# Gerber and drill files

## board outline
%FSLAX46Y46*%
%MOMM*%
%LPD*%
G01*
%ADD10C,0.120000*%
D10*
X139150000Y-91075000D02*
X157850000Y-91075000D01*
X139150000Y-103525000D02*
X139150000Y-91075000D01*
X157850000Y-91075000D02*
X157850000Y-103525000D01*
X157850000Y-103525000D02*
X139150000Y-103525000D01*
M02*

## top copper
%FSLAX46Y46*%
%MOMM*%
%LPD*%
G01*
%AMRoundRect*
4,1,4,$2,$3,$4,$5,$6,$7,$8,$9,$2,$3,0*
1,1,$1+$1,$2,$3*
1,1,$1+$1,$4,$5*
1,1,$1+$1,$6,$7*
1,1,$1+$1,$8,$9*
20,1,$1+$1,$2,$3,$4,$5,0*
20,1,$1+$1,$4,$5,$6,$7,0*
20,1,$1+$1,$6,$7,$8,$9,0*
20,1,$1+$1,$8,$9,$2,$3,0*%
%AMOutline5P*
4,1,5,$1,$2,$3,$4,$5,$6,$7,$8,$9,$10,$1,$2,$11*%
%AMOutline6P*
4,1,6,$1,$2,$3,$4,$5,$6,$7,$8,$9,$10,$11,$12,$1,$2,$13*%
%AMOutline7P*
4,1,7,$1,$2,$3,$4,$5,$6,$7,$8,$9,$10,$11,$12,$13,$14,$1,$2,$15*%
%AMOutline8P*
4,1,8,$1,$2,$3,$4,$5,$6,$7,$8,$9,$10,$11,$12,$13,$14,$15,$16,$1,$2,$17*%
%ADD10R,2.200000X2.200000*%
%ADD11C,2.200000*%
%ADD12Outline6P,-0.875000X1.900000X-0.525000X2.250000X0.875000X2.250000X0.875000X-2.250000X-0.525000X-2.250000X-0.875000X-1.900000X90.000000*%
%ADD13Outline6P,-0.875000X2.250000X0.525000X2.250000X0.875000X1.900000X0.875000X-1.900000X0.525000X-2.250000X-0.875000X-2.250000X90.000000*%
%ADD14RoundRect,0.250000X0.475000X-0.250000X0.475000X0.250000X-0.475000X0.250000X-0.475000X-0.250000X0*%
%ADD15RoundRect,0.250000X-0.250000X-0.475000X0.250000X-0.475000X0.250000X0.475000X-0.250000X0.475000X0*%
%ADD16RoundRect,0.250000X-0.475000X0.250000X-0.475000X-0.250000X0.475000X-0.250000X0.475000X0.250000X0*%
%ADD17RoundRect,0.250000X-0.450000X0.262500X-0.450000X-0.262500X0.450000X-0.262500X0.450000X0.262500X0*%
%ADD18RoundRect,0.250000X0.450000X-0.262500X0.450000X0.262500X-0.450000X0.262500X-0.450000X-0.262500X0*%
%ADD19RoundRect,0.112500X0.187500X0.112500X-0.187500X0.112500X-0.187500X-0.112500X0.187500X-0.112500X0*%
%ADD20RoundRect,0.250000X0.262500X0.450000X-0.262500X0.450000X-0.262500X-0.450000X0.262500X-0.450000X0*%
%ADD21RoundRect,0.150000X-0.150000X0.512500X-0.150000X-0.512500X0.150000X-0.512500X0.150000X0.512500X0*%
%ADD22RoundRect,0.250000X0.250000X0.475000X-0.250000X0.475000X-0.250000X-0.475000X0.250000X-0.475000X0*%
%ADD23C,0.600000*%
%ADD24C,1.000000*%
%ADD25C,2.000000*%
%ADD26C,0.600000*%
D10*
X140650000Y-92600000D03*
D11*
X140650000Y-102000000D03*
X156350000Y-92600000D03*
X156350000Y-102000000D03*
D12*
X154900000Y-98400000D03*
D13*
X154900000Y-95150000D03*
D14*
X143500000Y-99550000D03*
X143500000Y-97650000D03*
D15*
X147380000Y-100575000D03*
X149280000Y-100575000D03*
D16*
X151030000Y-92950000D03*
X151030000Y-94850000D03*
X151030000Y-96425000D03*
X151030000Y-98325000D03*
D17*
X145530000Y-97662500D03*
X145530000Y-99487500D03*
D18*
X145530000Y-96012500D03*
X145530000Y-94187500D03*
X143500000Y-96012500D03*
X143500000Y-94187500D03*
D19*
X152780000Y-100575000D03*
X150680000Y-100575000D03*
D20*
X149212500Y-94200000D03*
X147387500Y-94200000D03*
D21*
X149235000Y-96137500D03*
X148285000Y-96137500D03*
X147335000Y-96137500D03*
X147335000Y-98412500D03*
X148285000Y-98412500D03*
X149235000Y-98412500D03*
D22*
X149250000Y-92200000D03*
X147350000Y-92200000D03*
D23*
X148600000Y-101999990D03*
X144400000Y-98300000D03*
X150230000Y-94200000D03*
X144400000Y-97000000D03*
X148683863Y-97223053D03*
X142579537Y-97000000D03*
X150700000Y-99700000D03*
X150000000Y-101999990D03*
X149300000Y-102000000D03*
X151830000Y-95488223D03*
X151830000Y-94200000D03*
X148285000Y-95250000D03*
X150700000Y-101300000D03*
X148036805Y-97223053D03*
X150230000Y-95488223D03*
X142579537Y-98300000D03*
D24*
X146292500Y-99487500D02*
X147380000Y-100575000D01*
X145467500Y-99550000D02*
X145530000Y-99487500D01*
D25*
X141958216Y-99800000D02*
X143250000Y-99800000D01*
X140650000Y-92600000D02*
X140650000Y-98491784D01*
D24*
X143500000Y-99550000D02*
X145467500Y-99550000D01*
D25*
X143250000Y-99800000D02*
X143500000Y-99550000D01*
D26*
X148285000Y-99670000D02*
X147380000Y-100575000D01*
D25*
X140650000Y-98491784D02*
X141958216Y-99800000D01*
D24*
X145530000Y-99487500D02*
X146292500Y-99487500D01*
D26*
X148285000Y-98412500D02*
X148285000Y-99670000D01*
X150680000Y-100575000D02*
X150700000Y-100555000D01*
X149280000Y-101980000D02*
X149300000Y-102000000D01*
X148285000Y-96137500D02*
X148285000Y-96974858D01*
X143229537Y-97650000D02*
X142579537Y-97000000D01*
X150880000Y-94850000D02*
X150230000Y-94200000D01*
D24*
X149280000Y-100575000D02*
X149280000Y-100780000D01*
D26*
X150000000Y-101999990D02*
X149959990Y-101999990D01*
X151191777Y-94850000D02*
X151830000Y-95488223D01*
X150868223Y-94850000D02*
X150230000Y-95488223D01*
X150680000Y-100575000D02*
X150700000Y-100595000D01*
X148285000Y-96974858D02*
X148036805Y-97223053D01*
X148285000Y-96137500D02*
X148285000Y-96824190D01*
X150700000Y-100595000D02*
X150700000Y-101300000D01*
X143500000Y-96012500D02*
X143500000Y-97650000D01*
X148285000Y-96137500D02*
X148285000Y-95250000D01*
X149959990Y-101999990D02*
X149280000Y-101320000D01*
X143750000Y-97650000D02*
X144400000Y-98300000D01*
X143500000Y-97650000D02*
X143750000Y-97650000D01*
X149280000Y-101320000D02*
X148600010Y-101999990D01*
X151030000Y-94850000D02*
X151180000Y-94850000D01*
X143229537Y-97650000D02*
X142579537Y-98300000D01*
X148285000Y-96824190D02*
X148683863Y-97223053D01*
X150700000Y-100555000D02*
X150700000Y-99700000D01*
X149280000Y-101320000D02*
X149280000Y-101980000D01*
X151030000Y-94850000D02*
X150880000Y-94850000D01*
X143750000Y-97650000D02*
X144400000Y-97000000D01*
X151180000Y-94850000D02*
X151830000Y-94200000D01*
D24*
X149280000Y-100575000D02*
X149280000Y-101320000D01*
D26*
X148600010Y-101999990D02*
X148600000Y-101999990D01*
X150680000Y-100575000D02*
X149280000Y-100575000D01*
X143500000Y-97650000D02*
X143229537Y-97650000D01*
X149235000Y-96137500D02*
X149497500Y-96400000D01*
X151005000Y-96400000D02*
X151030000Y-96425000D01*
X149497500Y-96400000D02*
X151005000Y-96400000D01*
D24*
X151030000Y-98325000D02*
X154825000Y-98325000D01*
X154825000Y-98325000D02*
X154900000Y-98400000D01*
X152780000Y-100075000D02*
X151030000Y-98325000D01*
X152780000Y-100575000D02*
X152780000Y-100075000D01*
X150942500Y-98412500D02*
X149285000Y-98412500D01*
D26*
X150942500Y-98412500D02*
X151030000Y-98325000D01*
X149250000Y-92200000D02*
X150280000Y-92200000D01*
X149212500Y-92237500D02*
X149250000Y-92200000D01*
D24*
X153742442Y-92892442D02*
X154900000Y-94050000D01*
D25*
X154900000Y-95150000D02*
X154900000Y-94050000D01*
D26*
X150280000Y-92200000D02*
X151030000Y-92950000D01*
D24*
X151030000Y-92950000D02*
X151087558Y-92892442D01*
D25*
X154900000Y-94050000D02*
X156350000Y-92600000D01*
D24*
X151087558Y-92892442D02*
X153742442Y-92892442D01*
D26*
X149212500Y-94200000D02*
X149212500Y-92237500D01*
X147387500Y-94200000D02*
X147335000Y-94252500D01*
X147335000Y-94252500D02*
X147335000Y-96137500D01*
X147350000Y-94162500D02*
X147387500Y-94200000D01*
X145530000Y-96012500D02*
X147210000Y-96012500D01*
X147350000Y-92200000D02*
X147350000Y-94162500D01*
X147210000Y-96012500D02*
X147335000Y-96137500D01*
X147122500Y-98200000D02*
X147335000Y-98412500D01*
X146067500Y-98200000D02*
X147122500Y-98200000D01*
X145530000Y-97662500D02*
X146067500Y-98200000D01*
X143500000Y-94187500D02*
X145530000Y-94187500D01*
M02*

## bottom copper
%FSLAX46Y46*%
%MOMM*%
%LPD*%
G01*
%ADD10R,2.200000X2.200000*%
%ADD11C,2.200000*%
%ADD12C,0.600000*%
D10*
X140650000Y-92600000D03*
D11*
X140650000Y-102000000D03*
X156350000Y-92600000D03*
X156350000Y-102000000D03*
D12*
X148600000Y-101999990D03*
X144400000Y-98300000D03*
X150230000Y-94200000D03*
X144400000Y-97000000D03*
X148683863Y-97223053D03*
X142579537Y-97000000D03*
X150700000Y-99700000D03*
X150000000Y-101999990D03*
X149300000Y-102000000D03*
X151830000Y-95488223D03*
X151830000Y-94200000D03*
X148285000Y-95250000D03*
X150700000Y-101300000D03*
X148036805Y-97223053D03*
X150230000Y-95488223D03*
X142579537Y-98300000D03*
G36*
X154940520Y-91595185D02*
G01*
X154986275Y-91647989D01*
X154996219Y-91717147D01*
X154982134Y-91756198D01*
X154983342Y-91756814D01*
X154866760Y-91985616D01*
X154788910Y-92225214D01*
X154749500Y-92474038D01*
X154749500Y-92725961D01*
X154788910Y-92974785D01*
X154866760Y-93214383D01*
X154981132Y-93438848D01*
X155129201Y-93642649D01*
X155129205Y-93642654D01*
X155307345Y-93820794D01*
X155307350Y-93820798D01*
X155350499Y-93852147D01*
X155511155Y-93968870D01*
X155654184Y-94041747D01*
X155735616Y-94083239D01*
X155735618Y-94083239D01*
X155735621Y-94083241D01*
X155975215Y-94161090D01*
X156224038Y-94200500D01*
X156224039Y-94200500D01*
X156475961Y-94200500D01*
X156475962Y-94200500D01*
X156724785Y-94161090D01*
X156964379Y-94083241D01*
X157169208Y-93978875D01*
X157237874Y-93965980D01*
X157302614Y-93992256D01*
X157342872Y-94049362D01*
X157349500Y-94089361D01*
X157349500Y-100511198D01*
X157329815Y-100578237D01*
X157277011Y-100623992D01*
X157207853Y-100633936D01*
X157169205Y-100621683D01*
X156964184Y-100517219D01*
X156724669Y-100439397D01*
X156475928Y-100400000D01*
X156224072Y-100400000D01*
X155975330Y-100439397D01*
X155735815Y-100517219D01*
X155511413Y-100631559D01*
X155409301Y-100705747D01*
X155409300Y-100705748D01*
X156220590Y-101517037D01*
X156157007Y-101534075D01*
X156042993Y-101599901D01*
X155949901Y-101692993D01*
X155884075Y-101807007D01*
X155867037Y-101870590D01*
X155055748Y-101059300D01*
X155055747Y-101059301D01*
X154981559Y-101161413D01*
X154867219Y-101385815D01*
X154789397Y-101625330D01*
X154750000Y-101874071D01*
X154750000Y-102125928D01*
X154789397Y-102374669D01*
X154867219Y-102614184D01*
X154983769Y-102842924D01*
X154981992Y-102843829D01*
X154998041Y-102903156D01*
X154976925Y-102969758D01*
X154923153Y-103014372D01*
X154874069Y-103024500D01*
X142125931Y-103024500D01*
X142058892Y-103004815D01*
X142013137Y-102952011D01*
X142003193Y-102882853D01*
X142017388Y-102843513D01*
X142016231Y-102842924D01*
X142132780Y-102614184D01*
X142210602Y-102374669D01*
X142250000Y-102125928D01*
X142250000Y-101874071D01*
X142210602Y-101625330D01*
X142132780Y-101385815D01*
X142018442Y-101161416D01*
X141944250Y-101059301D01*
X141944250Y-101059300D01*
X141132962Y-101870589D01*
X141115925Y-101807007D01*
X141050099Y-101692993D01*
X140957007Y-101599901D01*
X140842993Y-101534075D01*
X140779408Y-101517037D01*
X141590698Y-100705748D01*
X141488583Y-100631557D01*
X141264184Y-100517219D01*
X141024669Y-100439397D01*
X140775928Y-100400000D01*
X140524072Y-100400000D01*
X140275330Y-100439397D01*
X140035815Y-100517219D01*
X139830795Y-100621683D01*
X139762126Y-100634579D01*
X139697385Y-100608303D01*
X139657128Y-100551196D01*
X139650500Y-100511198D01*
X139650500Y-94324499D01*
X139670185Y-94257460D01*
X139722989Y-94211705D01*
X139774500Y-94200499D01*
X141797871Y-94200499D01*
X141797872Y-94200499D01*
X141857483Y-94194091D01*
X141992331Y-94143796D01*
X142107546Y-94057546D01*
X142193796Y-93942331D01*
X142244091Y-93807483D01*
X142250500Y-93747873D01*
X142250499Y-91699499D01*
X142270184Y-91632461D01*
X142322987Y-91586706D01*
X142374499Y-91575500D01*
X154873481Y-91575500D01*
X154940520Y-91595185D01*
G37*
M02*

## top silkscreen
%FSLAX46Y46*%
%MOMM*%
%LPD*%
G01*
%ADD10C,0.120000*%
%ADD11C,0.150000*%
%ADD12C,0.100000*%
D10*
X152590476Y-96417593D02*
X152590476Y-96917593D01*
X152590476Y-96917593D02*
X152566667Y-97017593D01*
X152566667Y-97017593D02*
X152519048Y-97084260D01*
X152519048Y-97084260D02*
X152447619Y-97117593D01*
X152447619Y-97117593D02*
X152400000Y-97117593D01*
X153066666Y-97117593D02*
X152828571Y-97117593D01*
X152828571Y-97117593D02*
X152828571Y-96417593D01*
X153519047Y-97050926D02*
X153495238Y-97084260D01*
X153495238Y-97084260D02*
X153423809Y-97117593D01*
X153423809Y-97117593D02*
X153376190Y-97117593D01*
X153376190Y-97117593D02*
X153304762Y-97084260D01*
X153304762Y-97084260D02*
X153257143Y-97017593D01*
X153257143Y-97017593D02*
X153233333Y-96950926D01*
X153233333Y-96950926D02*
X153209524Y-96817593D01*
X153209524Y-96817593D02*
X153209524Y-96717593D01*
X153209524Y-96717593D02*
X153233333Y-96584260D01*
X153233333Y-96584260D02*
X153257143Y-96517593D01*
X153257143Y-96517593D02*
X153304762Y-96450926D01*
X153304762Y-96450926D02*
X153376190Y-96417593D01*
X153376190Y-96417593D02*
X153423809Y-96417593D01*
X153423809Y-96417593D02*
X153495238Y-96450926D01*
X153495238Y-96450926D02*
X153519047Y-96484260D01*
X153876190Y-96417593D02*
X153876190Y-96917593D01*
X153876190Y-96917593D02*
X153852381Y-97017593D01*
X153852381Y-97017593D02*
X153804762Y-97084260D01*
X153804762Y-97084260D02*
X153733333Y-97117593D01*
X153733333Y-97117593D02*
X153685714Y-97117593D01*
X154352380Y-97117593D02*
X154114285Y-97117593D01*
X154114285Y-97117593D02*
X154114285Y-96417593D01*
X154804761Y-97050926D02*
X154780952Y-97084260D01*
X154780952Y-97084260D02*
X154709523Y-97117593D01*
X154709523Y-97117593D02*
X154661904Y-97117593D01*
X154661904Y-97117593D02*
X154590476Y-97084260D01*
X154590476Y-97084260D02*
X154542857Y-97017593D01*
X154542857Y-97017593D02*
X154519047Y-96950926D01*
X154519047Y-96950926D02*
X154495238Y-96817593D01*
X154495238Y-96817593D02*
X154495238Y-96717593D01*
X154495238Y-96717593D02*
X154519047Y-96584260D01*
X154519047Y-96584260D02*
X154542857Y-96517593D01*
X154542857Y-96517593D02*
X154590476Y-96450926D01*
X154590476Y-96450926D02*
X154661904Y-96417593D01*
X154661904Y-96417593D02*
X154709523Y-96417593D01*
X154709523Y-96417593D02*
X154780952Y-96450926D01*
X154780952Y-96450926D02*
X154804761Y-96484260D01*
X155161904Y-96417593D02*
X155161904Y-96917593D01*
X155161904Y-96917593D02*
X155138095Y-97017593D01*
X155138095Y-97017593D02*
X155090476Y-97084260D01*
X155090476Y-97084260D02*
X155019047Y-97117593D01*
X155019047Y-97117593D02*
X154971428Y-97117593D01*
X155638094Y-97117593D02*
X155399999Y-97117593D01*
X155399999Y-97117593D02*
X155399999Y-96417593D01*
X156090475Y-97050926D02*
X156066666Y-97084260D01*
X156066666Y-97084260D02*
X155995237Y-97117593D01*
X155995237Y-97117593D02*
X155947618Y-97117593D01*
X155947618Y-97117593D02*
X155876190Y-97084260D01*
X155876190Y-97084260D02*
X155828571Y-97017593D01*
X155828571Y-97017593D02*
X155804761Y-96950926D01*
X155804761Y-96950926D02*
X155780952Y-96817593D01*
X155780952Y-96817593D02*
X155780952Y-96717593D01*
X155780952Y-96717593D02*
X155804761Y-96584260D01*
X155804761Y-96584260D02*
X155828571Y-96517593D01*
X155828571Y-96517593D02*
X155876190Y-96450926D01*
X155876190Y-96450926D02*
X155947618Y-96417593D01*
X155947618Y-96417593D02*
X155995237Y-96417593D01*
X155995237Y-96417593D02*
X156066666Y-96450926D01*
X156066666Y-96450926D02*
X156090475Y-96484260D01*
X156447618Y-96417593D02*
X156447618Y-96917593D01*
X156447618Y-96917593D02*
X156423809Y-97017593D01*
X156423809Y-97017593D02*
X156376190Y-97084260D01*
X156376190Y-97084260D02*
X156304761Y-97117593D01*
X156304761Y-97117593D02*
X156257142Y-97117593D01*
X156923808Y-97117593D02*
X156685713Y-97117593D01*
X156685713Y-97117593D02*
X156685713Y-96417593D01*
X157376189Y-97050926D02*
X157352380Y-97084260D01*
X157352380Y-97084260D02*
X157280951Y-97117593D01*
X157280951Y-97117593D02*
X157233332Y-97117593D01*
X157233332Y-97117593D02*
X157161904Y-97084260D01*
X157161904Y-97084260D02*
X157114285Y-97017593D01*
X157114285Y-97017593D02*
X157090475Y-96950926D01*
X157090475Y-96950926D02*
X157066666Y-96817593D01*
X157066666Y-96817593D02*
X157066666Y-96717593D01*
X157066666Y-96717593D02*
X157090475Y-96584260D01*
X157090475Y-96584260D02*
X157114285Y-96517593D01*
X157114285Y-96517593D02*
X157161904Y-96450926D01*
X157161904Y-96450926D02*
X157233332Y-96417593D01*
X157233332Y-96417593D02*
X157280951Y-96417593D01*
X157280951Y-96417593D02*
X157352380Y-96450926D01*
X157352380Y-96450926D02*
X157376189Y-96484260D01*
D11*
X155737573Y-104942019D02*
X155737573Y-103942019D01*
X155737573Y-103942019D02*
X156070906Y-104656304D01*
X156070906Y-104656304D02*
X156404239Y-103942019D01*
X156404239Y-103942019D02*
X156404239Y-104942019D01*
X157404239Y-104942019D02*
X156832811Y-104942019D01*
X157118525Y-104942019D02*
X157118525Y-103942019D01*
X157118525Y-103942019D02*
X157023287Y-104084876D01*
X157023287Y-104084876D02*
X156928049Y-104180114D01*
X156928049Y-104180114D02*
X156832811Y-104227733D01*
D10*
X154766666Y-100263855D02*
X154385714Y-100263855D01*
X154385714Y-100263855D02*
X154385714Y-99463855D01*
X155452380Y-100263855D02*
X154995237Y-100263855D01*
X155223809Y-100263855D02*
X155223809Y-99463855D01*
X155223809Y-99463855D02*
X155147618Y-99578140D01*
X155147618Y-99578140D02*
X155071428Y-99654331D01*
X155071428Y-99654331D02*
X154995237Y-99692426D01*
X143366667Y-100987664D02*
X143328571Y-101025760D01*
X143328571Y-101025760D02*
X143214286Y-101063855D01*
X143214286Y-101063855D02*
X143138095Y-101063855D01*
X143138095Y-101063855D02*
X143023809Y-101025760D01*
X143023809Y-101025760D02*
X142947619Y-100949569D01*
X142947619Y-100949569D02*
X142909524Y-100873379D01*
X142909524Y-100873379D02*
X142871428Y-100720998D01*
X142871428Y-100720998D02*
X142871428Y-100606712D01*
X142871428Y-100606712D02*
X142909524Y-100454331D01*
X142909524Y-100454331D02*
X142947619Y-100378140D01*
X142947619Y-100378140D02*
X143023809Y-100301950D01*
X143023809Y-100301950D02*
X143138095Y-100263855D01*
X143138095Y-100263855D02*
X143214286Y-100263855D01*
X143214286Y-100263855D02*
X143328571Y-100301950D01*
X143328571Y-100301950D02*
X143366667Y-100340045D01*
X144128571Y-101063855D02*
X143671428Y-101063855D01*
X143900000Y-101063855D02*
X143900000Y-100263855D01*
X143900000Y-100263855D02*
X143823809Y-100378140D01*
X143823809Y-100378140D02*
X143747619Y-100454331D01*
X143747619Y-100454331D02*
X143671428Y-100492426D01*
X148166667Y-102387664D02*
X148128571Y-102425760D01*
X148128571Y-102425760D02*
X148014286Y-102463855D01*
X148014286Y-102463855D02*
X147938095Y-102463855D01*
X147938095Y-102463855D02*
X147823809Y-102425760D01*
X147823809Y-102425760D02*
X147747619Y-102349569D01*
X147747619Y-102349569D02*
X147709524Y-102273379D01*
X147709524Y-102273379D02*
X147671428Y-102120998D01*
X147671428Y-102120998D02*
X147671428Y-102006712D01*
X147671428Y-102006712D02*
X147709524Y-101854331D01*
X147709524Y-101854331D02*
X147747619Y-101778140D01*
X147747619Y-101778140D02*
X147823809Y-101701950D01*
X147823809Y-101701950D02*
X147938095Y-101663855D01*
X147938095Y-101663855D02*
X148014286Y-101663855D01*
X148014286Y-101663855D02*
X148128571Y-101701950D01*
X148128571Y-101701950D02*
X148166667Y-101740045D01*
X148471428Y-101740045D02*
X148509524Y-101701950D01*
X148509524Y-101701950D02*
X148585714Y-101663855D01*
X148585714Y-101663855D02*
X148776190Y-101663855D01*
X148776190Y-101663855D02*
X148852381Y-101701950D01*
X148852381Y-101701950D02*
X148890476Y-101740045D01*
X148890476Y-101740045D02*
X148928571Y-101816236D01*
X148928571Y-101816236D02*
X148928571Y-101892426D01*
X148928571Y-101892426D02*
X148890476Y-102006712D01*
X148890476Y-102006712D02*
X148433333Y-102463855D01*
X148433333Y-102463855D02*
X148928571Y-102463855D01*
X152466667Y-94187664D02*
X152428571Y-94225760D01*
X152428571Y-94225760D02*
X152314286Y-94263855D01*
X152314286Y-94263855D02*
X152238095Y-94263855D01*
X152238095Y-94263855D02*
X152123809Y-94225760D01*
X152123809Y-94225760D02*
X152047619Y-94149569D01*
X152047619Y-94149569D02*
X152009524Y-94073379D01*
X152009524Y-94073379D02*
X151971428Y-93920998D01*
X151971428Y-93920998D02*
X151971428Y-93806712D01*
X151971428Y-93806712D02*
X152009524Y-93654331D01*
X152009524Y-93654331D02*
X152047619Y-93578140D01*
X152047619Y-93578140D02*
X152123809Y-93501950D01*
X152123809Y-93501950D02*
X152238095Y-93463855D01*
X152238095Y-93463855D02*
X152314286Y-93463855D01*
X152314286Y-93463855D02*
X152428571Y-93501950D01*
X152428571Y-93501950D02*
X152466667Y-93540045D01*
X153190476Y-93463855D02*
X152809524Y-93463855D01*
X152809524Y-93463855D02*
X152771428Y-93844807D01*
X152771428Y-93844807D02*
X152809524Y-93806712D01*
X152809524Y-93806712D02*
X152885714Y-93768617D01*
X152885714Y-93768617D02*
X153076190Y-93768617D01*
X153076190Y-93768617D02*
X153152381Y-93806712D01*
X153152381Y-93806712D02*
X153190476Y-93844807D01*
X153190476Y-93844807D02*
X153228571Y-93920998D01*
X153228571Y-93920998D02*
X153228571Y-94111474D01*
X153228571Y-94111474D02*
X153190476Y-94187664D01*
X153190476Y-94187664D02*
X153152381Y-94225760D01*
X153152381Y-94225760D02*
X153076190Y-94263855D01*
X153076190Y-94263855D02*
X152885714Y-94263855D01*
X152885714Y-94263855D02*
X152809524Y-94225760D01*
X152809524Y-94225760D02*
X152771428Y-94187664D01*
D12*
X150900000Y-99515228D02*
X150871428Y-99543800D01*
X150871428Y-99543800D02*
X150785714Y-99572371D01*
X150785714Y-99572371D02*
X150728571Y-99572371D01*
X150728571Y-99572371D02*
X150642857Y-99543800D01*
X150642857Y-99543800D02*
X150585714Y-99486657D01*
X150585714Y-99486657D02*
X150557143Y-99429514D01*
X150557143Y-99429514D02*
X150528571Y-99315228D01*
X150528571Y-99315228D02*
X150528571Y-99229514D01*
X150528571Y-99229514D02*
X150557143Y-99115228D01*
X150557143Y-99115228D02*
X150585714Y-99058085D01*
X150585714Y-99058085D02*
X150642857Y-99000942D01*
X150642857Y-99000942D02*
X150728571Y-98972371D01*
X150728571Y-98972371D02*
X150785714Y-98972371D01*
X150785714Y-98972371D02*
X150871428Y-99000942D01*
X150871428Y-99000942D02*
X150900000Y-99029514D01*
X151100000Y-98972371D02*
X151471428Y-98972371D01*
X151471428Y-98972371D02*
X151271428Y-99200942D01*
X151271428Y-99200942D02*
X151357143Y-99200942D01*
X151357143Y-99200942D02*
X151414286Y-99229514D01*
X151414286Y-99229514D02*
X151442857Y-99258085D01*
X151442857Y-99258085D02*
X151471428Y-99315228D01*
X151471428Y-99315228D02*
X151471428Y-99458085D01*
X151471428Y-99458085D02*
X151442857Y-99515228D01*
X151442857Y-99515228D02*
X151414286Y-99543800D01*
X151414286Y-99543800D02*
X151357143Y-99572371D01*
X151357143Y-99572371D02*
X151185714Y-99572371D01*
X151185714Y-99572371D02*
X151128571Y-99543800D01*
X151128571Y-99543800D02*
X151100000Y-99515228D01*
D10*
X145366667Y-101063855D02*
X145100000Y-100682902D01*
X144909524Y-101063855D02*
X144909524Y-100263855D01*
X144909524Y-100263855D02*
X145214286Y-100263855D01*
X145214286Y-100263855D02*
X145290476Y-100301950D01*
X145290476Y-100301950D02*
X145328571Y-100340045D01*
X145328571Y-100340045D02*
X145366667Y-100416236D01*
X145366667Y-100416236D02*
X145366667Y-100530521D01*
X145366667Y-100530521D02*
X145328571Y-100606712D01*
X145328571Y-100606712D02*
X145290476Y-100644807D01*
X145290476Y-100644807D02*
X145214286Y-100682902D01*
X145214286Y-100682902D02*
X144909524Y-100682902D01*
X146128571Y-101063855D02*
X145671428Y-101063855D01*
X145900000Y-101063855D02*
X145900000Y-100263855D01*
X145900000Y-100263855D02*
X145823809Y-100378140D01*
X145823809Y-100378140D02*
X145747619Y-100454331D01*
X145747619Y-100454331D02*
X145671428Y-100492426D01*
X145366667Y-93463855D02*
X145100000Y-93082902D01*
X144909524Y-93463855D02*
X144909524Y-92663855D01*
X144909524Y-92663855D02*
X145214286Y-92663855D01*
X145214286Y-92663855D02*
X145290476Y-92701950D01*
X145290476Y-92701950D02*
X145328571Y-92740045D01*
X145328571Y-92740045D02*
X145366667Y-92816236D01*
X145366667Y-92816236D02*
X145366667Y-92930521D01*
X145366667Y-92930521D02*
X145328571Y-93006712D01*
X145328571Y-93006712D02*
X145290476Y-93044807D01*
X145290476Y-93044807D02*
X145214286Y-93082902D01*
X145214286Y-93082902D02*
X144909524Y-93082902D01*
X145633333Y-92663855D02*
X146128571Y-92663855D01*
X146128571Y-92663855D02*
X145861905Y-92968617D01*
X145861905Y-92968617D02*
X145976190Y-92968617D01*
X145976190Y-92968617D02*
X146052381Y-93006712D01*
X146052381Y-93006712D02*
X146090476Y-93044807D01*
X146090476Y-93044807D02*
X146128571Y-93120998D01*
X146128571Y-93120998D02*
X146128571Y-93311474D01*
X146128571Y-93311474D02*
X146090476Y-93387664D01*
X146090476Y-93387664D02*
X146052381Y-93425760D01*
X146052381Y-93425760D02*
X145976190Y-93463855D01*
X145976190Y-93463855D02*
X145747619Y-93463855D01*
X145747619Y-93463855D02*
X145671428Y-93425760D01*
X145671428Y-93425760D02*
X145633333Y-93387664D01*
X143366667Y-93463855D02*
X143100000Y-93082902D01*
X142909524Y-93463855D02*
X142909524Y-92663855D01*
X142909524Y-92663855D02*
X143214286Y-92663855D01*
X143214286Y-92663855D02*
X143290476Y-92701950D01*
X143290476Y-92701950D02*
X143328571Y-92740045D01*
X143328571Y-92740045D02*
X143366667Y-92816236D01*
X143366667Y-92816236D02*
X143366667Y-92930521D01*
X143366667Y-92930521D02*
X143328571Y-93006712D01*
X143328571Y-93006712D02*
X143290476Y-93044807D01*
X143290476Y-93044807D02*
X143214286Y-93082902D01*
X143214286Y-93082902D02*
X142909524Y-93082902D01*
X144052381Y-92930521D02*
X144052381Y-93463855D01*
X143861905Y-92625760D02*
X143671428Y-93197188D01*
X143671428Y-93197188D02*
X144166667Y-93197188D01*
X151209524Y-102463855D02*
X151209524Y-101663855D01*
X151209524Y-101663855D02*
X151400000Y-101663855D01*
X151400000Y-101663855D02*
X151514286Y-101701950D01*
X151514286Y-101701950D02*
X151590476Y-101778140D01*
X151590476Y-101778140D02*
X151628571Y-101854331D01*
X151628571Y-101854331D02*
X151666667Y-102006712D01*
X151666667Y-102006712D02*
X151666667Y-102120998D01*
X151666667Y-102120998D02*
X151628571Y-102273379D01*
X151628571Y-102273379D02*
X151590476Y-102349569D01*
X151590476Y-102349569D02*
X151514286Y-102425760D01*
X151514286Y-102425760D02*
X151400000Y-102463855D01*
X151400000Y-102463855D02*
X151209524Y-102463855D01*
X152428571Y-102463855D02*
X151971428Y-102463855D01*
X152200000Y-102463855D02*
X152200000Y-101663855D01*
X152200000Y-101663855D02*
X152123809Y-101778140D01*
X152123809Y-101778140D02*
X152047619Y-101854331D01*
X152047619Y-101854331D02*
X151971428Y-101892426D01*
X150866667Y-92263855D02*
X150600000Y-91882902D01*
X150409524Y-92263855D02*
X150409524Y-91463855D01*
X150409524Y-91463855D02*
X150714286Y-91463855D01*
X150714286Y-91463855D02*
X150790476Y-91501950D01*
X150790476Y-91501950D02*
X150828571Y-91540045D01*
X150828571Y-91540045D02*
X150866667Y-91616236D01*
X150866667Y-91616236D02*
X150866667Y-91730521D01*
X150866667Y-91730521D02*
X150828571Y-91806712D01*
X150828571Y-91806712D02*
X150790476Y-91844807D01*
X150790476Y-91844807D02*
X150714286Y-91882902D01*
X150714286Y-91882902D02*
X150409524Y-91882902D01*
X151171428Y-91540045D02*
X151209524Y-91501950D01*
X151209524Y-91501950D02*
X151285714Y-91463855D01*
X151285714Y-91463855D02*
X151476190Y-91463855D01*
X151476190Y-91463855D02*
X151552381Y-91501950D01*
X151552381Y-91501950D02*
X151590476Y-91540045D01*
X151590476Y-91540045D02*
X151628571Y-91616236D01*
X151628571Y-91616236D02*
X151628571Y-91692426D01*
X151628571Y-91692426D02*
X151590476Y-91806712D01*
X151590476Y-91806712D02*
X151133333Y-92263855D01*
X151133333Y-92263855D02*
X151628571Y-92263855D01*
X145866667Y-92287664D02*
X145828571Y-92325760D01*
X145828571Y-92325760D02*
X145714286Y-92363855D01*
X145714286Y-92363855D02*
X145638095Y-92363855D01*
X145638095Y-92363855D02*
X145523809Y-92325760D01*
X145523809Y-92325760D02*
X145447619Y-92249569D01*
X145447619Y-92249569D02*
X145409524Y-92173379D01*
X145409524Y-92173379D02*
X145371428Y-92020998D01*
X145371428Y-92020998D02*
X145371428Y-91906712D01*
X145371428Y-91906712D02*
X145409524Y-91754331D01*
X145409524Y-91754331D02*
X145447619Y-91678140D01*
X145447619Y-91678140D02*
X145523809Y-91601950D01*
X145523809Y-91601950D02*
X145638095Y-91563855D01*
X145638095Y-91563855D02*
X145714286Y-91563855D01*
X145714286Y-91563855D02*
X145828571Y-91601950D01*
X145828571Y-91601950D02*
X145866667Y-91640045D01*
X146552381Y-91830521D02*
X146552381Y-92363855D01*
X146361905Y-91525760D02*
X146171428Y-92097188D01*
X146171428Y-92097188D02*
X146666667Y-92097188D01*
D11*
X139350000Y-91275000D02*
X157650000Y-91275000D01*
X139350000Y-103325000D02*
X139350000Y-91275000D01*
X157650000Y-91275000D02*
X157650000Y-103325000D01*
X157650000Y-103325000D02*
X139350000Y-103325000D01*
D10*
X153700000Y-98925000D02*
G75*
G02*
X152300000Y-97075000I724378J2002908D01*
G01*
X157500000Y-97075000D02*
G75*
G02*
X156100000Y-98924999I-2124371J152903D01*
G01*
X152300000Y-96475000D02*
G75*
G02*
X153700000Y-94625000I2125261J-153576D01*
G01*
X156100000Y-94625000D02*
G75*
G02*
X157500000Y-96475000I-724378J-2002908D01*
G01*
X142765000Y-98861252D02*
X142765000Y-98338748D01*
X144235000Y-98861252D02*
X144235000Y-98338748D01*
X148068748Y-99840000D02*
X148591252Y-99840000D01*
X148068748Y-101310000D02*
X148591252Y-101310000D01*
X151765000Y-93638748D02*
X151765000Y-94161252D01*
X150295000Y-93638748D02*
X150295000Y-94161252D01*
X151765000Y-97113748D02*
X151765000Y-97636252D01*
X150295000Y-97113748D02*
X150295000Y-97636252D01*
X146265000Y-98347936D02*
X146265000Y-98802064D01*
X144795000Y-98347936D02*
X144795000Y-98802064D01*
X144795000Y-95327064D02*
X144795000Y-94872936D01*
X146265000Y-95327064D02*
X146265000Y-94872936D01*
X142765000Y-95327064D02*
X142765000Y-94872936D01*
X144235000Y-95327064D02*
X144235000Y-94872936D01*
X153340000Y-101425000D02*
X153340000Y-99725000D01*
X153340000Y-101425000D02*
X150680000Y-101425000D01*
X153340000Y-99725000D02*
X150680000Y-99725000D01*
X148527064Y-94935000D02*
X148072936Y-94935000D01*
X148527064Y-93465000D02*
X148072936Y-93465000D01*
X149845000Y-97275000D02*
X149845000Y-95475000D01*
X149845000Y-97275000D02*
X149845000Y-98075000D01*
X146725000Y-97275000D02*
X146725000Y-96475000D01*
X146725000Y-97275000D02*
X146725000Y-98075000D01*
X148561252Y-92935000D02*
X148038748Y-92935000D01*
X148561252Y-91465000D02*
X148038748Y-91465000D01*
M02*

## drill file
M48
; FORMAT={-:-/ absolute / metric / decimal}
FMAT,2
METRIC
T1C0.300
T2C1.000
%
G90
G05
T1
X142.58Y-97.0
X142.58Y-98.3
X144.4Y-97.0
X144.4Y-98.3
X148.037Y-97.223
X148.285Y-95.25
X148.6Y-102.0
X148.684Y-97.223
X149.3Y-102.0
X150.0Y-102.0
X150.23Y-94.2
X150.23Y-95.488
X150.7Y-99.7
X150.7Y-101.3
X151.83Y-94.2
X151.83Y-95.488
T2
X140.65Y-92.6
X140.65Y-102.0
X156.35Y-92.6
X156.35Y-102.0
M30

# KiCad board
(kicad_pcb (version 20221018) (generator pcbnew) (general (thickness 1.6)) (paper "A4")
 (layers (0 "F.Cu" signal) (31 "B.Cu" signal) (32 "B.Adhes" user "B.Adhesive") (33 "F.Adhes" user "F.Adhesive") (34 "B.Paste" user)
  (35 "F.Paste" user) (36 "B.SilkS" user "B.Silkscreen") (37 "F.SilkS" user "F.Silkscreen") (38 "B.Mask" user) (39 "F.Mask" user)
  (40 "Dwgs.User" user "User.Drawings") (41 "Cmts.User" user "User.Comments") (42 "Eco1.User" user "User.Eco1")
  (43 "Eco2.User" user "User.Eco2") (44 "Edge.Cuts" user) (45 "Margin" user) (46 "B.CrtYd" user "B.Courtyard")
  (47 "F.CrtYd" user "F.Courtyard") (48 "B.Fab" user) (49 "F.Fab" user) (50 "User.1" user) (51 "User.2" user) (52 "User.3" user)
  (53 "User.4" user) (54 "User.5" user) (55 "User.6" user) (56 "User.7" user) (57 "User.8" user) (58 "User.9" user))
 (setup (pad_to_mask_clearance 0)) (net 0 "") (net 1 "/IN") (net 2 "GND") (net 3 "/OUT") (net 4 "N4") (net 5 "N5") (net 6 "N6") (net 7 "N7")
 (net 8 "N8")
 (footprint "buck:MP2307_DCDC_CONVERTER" (layer "F.Cu") (at 140.65 92.6)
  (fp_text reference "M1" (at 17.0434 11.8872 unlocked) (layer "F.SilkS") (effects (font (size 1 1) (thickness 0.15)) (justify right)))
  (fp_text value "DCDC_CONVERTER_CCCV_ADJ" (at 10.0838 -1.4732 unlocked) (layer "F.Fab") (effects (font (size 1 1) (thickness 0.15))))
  (fp_line (start -1.3 -1.325) (end 17 -1.325) (stroke (width 0.15) (type solid)) (layer "F.SilkS"))
  (fp_line (start -1.3 10.725) (end -1.3 -1.325) (stroke (width 0.15) (type solid)) (layer "F.SilkS"))
  (fp_line (start 17 -1.325) (end 17 10.725) (stroke (width 0.15) (type solid)) (layer "F.SilkS"))
  (fp_line (start 17 10.725) (end -1.3 10.725) (stroke (width 0.15) (type solid)) (layer "F.SilkS"))
  (fp_line (start -1.5 -1.525) (end 17.2 -1.525) (stroke (width 0.12) (type solid)) (layer "Edge.Cuts"))
  (fp_line (start -1.5 10.925) (end -1.5 -1.525) (stroke (width 0.12) (type solid)) (layer "Edge.Cuts"))
  (fp_line (start 17.2 -1.525) (end 17.2 10.925) (stroke (width 0.12) (type solid)) (layer "Edge.Cuts"))
  (fp_line (start 17.2 10.925) (end -1.5 10.925) (stroke (width 0.12) (type solid)) (layer "Edge.Cuts"))
  (pad "1" thru_hole rect (at 0 0) (size 2.2 2.2) (drill 1) (layers "*.Cu" "*.Mask") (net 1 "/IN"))
  (pad "2" thru_hole circle (at 0 9.4) (size 2.2 2.2) (drill 1) (layers "*.Cu" "*.Mask") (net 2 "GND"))
  (pad "3" thru_hole circle (at 15.7 0) (size 2.2 2.2) (drill 1) (layers "*.Cu" "*.Mask") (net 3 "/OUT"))
  (pad "4" thru_hole circle (at 15.7 9.4) (size 2.2 2.2) (drill 1) (layers "*.Cu" "*.Mask") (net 2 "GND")))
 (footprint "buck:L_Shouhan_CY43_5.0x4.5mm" (layer "F.Cu") (at 154.9 96.775 90)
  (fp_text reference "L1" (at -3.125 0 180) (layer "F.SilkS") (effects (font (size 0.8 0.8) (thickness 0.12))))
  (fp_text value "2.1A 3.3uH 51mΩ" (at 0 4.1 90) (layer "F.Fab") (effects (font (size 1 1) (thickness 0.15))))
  (fp_arc (start -2.15 -1.2) (mid -1.432349 -2.173997) (end -0.3 -2.6) (stroke (width 0.12) (type solid)) (layer "F.SilkS"))
  (fp_arc (start -0.3 2.6) (mid -1.43235 2.173998) (end -2.15 1.2) (stroke (width 0.12) (type solid)) (layer "F.SilkS"))
  (fp_arc (start 0.3 -2.6) (mid 1.432241 -2.173855) (end 2.15 -1.2) (stroke (width 0.12) (type solid)) (layer "F.SilkS"))
  (fp_arc (start 2.15 1.2) (mid 1.432349 2.173997) (end 0.3 2.6) (stroke (width 0.12) (type solid)) (layer "F.SilkS"))
  (pad "1" smd roundrect (at -1.625 0 90) (size 1.75 4.5) (layers "F.Cu" "F.Paste" "F.Mask") (roundrect_rratio 0) (chamfer_ratio 0.2)
   (chamfer top_left bottom_left) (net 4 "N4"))
  (pad "2" smd roundrect (at 1.625 0 90) (size 1.75 4.5) (layers "F.Cu" "F.Paste" "F.Mask") (roundrect_rratio 0) (chamfer_ratio 0.2)
   (chamfer top_right bottom_right) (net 3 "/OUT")))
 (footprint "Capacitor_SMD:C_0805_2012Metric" (layer "F.Cu") (at 143.5 98.6 90)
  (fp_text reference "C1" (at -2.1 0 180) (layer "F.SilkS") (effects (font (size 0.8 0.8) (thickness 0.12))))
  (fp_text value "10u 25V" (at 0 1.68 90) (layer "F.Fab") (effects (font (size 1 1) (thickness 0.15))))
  (fp_line (start -0.261252 -0.735) (end 0.261252 -0.735) (stroke (width 0.12) (type solid)) (layer "F.SilkS"))
  (fp_line (start -0.261252 0.735) (end 0.261252 0.735) (stroke (width 0.12) (type solid)) (layer "F.SilkS"))
  (pad "1" smd roundrect (at -0.95 0 90) (size 1 1.45) (layers "F.Cu" "F.Paste" "F.Mask") (roundrect_rratio 0.25) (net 1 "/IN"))
  (pad "2" smd roundrect (at 0.95 0 90) (size 1 1.45) (layers "F.Cu" "F.Paste" "F.Mask") (roundrect_rratio 0.25) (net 2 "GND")))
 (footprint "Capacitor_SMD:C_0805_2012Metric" (layer "F.Cu") (at 148.33 100.575)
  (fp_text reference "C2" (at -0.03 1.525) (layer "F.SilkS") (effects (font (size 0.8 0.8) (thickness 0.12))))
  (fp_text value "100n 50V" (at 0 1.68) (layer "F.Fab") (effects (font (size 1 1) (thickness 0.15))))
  (fp_line (start -0.261252 -0.735) (end 0.261252 -0.735) (stroke (width 0.12) (type solid)) (layer "F.SilkS"))
  (fp_line (start -0.261252 0.735) (end 0.261252 0.735) (stroke (width 0.12) (type solid)) (layer "F.SilkS"))
  (pad "1" smd roundrect (at -0.95 0) (size 1 1.45) (layers "F.Cu" "F.Paste" "F.Mask") (roundrect_rratio 0.25) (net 1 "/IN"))
  (pad "2" smd roundrect (at 0.95 0) (size 1 1.45) (layers "F.Cu" "F.Paste" "F.Mask") (roundrect_rratio 0.25) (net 2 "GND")))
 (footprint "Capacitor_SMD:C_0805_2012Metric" (layer "F.Cu") (at 151.03 93.9 -90)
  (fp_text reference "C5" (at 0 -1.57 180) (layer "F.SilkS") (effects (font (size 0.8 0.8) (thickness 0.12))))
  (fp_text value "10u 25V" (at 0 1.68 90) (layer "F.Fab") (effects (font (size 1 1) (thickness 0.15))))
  (fp_line (start -0.261252 -0.735) (end 0.261252 -0.735) (stroke (width 0.12) (type solid)) (layer "F.SilkS"))
  (fp_line (start -0.261252 0.735) (end 0.261252 0.735) (stroke (width 0.12) (type solid)) (layer "F.SilkS"))
  (pad "1" smd roundrect (at -0.95 0 270) (size 1 1.45) (layers "F.Cu" "F.Paste" "F.Mask") (roundrect_rratio 0.25) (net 3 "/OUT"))
  (pad "2" smd roundrect (at 0.95 0 270) (size 1 1.45) (layers "F.Cu" "F.Paste" "F.Mask") (roundrect_rratio 0.25) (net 2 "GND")))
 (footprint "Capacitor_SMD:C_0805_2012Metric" (layer "F.Cu") (at 151.03 97.375 -90)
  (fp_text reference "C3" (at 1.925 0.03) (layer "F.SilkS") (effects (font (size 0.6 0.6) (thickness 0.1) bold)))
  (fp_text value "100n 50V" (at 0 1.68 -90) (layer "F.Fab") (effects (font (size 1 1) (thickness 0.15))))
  (fp_line (start -0.261252 -0.735) (end 0.261252 -0.735) (stroke (width 0.12) (type solid)) (layer "F.SilkS"))
  (fp_line (start -0.261252 0.735) (end 0.261252 0.735) (stroke (width 0.12) (type solid)) (layer "F.SilkS"))
  (pad "1" smd roundrect (at -0.95 0 270) (size 1 1.45) (layers "F.Cu" "F.Paste" "F.Mask") (roundrect_rratio 0.25) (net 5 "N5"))
  (pad "2" smd roundrect (at 0.95 0 270) (size 1 1.45) (layers "F.Cu" "F.Paste" "F.Mask") (roundrect_rratio 0.25) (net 4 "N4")))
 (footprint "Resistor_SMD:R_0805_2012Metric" (layer "F.Cu") (at 145.53 98.575 -90)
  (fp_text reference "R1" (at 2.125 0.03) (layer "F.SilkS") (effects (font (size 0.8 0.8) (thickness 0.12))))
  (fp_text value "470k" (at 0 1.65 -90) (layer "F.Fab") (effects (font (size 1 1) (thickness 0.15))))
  (fp_line (start -0.227064 -0.735) (end 0.227064 -0.735) (stroke (width 0.12) (type solid)) (layer "F.SilkS"))
  (fp_line (start -0.227064 0.735) (end 0.227064 0.735) (stroke (width 0.12) (type solid)) (layer "F.SilkS"))
  (pad "1" smd roundrect (at -0.9125 0 270) (size 1.025 1.4) (layers "F.Cu" "F.Paste" "F.Mask") (roundrect_rratio 0.243902439) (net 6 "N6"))
  (pad "2" smd roundrect (at 0.9125 0 270) (size 1.025 1.4) (layers "F.Cu" "F.Paste" "F.Mask") (roundrect_rratio 0.243902439) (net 1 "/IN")))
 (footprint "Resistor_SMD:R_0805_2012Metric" (layer "F.Cu") (at 145.53 95.1 90)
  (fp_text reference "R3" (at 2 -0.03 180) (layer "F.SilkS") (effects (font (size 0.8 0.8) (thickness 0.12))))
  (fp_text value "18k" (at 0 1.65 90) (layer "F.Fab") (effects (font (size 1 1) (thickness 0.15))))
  (fp_line (start -0.227064 -0.735) (end 0.227064 -0.735) (stroke (width 0.12) (type solid)) (layer "F.SilkS"))
  (fp_line (start -0.227064 0.735) (end 0.227064 0.735) (stroke (width 0.12) (type solid)) (layer "F.SilkS"))
  (pad "1" smd roundrect (at -0.9125 0 90) (size 1.025 1.4) (layers "F.Cu" "F.Paste" "F.Mask") (roundrect_rratio 0.243902439) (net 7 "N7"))
  (pad "2" smd roundrect (at 0.9125 0 90) (size 1.025 1.4) (layers "F.Cu" "F.Paste" "F.Mask") (roundrect_rratio 0.243902439) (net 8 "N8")))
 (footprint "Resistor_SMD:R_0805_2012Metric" (layer "F.Cu") (at 143.5 95.1 90)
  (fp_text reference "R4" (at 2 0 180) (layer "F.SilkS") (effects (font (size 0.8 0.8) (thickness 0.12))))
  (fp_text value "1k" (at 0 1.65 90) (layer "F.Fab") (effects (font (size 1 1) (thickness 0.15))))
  (fp_line (start -0.227064 -0.735) (end 0.227064 -0.735) (stroke (width 0.12) (type solid)) (layer "F.SilkS"))
  (fp_line (start -0.227064 0.735) (end 0.227064 0.735) (stroke (width 0.12) (type solid)) (layer "F.SilkS"))
  (pad "1" smd roundrect (at -0.9125 0 90) (size 1.025 1.4) (layers "F.Cu" "F.Paste" "F.Mask") (roundrect_rratio 0.243902439) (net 2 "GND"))
  (pad "2" smd roundrect (at 0.9125 0 90) (size 1.025 1.4) (layers "F.Cu" "F.Paste" "F.Mask") (roundrect_rratio 0.243902439) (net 8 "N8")))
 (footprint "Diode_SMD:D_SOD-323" (layer "F.Cu") (at 151.73 100.575 180)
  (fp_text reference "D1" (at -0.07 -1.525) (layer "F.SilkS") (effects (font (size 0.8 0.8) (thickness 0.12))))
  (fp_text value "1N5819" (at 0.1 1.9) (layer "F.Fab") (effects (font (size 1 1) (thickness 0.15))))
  (fp_line (start -1.61 -0.85) (end -1.61 0.85) (stroke (width 0.12) (type solid)) (layer "F.SilkS"))
  (fp_line (start -1.61 -0.85) (end 1.05 -0.85) (stroke (width 0.12) (type solid)) (layer "F.SilkS"))
  (fp_line (start -1.61 0.85) (end 1.05 0.85) (stroke (width 0.12) (type solid)) (layer "F.SilkS"))
  (pad "1" smd roundrect (at -1.05 0 180) (size 0.6 0.45) (layers "F.Cu" "F.Paste" "F.Mask") (roundrect_rratio 0.25) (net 4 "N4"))
  (pad "2" smd roundrect (at 1.05 0 180) (size 0.6 0.45) (layers "F.Cu" "F.Paste" "F.Mask") (roundrect_rratio 0.25) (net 2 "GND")))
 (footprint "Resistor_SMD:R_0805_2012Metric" (layer "F.Cu") (at 148.3 94.2 180)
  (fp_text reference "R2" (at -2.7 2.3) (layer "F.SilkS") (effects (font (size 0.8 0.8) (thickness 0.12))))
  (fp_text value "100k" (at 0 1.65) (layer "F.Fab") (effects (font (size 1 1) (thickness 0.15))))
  (fp_line (start -0.227064 -0.735) (end 0.227064 -0.735) (stroke (width 0.12) (type solid)) (layer "F.SilkS"))
  (fp_line (start -0.227064 0.735) (end 0.227064 0.735) (stroke (width 0.12) (type solid)) (layer "F.SilkS"))
  (pad "1" smd roundrect (at -0.9125 0 180) (size 1.025 1.4) (layers "F.Cu" "F.Paste" "F.Mask") (roundrect_rratio 0.243902439)
   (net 3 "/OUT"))
  (pad "2" smd roundrect (at 0.9125 0 180) (size 1.025 1.4) (layers "F.Cu" "F.Paste" "F.Mask") (roundrect_rratio 0.243902439) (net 7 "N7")))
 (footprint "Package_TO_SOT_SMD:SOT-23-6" (layer "F.Cu") (at 148.285 97.275 -90)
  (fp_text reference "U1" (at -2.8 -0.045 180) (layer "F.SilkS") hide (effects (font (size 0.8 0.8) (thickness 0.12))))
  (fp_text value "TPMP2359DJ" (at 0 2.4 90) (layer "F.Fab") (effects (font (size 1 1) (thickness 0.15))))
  (fp_line (start 0 -1.56) (end -1.8 -1.56) (stroke (width 0.12) (type solid)) (layer "F.SilkS"))
  (fp_line (start 0 -1.56) (end 0.8 -1.56) (stroke (width 0.12) (type solid)) (layer "F.SilkS"))
  (fp_line (start 0 1.56) (end -0.8 1.56) (stroke (width 0.12) (type solid)) (layer "F.SilkS"))
  (fp_line (start 0 1.56) (end 0.8 1.56) (stroke (width 0.12) (type solid)) (layer "F.SilkS"))
  (pad "1" smd roundrect (at -1.1375 -0.95 270) (size 1.325 0.6) (layers "F.Cu" "F.Paste" "F.Mask") (roundrect_rratio 0.25) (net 5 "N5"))
  (pad "2" smd roundrect (at -1.1375 0 270) (size 1.325 0.6) (layers "F.Cu" "F.Paste" "F.Mask") (roundrect_rratio 0.25) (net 2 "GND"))
  (pad "3" smd roundrect (at -1.1375 0.95 270) (size 1.325 0.6) (layers "F.Cu" "F.Paste" "F.Mask") (roundrect_rratio 0.25) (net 7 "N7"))
  (pad "4" smd roundrect (at 1.1375 0.95 270) (size 1.325 0.6) (layers "F.Cu" "F.Paste" "F.Mask") (roundrect_rratio 0.25) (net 6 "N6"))
  (pad "5" smd roundrect (at 1.1375 0 270) (size 1.325 0.6) (layers "F.Cu" "F.Paste" "F.Mask") (roundrect_rratio 0.25) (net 1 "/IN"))
  (pad "6" smd roundrect (at 1.1375 -0.95 270) (size 1.325 0.6) (layers "F.Cu" "F.Paste" "F.Mask") (roundrect_rratio 0.25) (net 4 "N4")))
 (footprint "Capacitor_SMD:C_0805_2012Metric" (layer "F.Cu") (at 148.3 92.2 180)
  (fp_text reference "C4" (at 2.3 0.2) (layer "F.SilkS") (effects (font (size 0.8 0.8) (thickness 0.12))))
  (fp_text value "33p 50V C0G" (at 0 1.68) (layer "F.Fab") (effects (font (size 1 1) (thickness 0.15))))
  (fp_line (start -0.261252 -0.735) (end 0.261252 -0.735) (stroke (width 0.12) (type solid)) (layer "F.SilkS"))
  (fp_line (start -0.261252 0.735) (end 0.261252 0.735) (stroke (width 0.12) (type solid)) (layer "F.SilkS"))
  (pad "1" smd roundrect (at -0.95 0 180) (size 1 1.45) (layers "F.Cu" "F.Paste" "F.Mask") (roundrect_rratio 0.25) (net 3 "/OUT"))
  (pad "2" smd roundrect (at 0.95 0 180) (size 1 1.45) (layers "F.Cu" "F.Paste" "F.Mask") (roundrect_rratio 0.25) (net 7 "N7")))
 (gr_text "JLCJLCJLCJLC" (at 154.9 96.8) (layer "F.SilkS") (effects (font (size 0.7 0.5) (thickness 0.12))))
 (segment (start 146.2925 99.4875) (end 147.38 100.575) (width 1) (layer "F.Cu") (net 1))
 (segment (start 145.4675 99.55) (end 145.53 99.4875) (width 1) (layer "F.Cu") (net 1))
 (segment (start 141.958216 99.8) (end 143.25 99.8) (width 2) (layer "F.Cu") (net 1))
 (segment (start 140.65 92.6) (end 140.65 98.491784) (width 2) (layer "F.Cu") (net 1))
 (segment (start 143.5 99.55) (end 145.4675 99.55) (width 1) (layer "F.Cu") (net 1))
 (segment (start 143.25 99.8) (end 143.5 99.55) (width 2) (layer "F.Cu") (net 1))
 (segment (start 148.285 99.67) (end 147.38 100.575) (width 0.6) (layer "F.Cu") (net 1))
 (segment (start 140.65 98.491784) (end 141.958216 99.8) (width 2) (layer "F.Cu") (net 1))
 (segment (start 145.53 99.4875) (end 146.2925 99.4875) (width 1) (layer "F.Cu") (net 1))
 (segment (start 148.285 98.4125) (end 148.285 99.67) (width 0.6) (layer "F.Cu") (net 1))
 (segment (start 150.68 100.575) (end 150.7 100.555) (width 0.6) (layer "F.Cu") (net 2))
 (segment (start 149.28 101.98) (end 149.3 102) (width 0.6) (layer "F.Cu") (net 2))
 (segment (start 148.285 96.1375) (end 148.285 96.974858) (width 0.6) (layer "F.Cu") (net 2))
 (segment (start 143.229537 97.65) (end 142.579537 97) (width 0.6) (layer "F.Cu") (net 2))
 (segment (start 150.88 94.85) (end 150.23 94.2) (width 0.6) (layer "F.Cu") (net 2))
 (segment (start 149.28 100.575) (end 149.28 100.78) (width 1) (layer "F.Cu") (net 2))
 (segment (start 150 101.99999) (end 149.95999 101.99999) (width 0.6) (layer "F.Cu") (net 2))
 (segment (start 151.191777 94.85) (end 151.83 95.488223) (width 0.6) (layer "F.Cu") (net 2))
 (segment (start 150.868223 94.85) (end 150.23 95.488223) (width 0.6) (layer "F.Cu") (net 2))
 (segment (start 150.68 100.575) (end 150.7 100.595) (width 0.6) (layer "F.Cu") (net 2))
 (segment (start 148.285 96.974858) (end 148.036805 97.223053) (width 0.6) (layer "F.Cu") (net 2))
 (segment (start 148.285 96.1375) (end 148.285 96.82419) (width 0.6) (layer "F.Cu") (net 2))
 (segment (start 150.7 100.595) (end 150.7 101.3) (width 0.6) (layer "F.Cu") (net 2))
 (segment (start 143.5 96.0125) (end 143.5 97.65) (width 0.6) (layer "F.Cu") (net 2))
 (segment (start 148.285 96.1375) (end 148.285 95.25) (width 0.6) (layer "F.Cu") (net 2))
 (segment (start 149.95999 101.99999) (end 149.28 101.32) (width 0.6) (layer "F.Cu") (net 2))
 (segment (start 143.75 97.65) (end 144.4 98.3) (width 0.6) (layer "F.Cu") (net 2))
 (segment (start 143.5 97.65) (end 143.75 97.65) (width 0.6) (layer "F.Cu") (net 2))
 (segment (start 149.28 101.32) (end 148.60001 101.99999) (width 0.6) (layer "F.Cu") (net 2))
 (segment (start 151.03 94.85) (end 151.18 94.85) (width 0.6) (layer "F.Cu") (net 2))
 (segment (start 143.229537 97.65) (end 142.579537 98.3) (width 0.6) (layer "F.Cu") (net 2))
 (segment (start 148.285 96.82419) (end 148.683863 97.223053) (width 0.6) (layer "F.Cu") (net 2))
 (segment (start 150.7 100.555) (end 150.7 99.7) (width 0.6) (layer "F.Cu") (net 2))
 (segment (start 149.28 101.32) (end 149.28 101.98) (width 0.6) (layer "F.Cu") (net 2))
 (segment (start 151.03 94.85) (end 150.88 94.85) (width 0.6) (layer "F.Cu") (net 2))
 (segment (start 143.75 97.65) (end 144.4 97) (width 0.6) (layer "F.Cu") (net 2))
 (segment (start 151.18 94.85) (end 151.83 94.2) (width 0.6) (layer "F.Cu") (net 2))
 (segment (start 149.28 100.575) (end 149.28 101.32) (width 1) (layer "F.Cu") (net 2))
 (segment (start 148.60001 101.99999) (end 148.6 101.99999) (width 0.6) (layer "F.Cu") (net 2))
 (segment (start 150.68 100.575) (end 149.28 100.575) (width 0.6) (layer "F.Cu") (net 2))
 (segment (start 143.5 97.65) (end 143.229537 97.65) (width 0.6) (layer "F.Cu") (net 2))
 (via (at 148.6 101.99999) (size 0.6) (drill 0.3) (layers "F.Cu" "B.Cu") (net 2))
 (via (at 144.4 98.3) (size 0.6) (drill 0.3) (layers "F.Cu" "B.Cu") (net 2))
 (via (at 150.23 94.2) (size 0.6) (drill 0.3) (layers "F.Cu" "B.Cu") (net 2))
 (via (at 144.4 97) (size 0.6) (drill 0.3) (layers "F.Cu" "B.Cu") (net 2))
 (via (at 148.683863 97.223053) (size 0.6) (drill 0.3) (layers "F.Cu" "B.Cu") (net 2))
 (via (at 142.579537 97) (size 0.6) (drill 0.3) (layers "F.Cu" "B.Cu") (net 2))
 (via (at 150.7 99.7) (size 0.6) (drill 0.3) (layers "F.Cu" "B.Cu") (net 2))
 (via (at 150 101.99999) (size 0.6) (drill 0.3) (layers "F.Cu" "B.Cu") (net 2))
 (via (at 149.3 102) (size 0.6) (drill 0.3) (layers "F.Cu" "B.Cu") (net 2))
 (via (at 151.83 95.488223) (size 0.6) (drill 0.3) (layers "F.Cu" "B.Cu") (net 2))
 (via (at 151.83 94.2) (size 0.6) (drill 0.3) (layers "F.Cu" "B.Cu") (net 2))
 (via (at 148.285 95.25) (size 0.6) (drill 0.3) (layers "F.Cu" "B.Cu") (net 2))
 (via (at 150.7 101.3) (size 0.6) (drill 0.3) (layers "F.Cu" "B.Cu") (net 2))
 (via (at 148.036805 97.223053) (size 0.6) (drill 0.3) (layers "F.Cu" "B.Cu") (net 2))
 (via (at 150.23 95.488223) (size 0.6) (drill 0.3) (layers "F.Cu" "B.Cu") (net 2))
 (via (at 142.579537 98.3) (size 0.6) (drill 0.3) (layers "F.Cu" "B.Cu") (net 2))
 (segment (start 149.235 96.1375) (end 149.4975 96.4) (width 0.6) (layer "F.Cu") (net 5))
 (segment (start 151.005 96.4) (end 151.03 96.425) (width 0.6) (layer "F.Cu") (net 5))
 (segment (start 149.4975 96.4) (end 151.005 96.4) (width 0.6) (layer "F.Cu") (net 5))
 (segment (start 151.03 98.325) (end 154.825 98.325) (width 1) (layer "F.Cu") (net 4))
 (segment (start 154.825 98.325) (end 154.9 98.4) (width 1) (layer "F.Cu") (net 4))
 (segment (start 152.78 100.075) (end 151.03 98.325) (width 1) (layer "F.Cu") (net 4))
 (segment (start 152.78 100.575) (end 152.78 100.075) (width 1) (layer "F.Cu") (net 4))
 (segment (start 150.9425 98.4125) (end 149.285 98.4125) (width 1) (layer "F.Cu") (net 4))
 (segment (start 150.9425 98.4125) (end 151.03 98.325) (width 0.6) (layer "F.Cu") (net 4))
 (segment (start 149.25 92.2) (end 150.28 92.2) (width 0.6) (layer "F.Cu") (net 3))
 (segment (start 149.2125 92.2375) (end 149.25 92.2) (width 0.6) (layer "F.Cu") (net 3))
 (segment (start 153.742442 92.892442) (end 154.9 94.05) (width 1) (layer "F.Cu") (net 3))
 (segment (start 154.9 95.15) (end 154.9 94.05) (width 2) (layer "F.Cu") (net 3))
 (segment (start 150.28 92.2) (end 151.03 92.95) (width 0.6) (layer "F.Cu") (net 3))
 (segment (start 151.03 92.95) (end 151.087558 92.892442) (width 1) (layer "F.Cu") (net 3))
 (segment (start 154.9 94.05) (end 156.35 92.6) (width 2) (layer "F.Cu") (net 3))
 (segment (start 151.087558 92.892442) (end 153.742442 92.892442) (width 1) (layer "F.Cu") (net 3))
 (segment (start 149.2125 94.2) (end 149.2125 92.2375) (width 0.6) (layer "F.Cu") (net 3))
 (segment (start 147.3875 94.2) (end 147.335 94.2525) (width 0.6) (layer "F.Cu") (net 7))
 (segment (start 147.335 94.2525) (end 147.335 96.1375) (width 0.6) (layer "F.Cu") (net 7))
 (segment (start 147.35 94.1625) (end 147.3875 94.2) (width 0.6) (layer "F.Cu") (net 7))
 (segment (start 145.53 96.0125) (end 147.21 96.0125) (width 0.6) (layer "F.Cu") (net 7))
 (segment (start 147.35 92.2) (end 147.35 94.1625) (width 0.6) (layer "F.Cu") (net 7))
 (segment (start 147.21 96.0125) (end 147.335 96.1375) (width 0.6) (layer "F.Cu") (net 7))
 (segment (start 147.1225 98.2) (end 147.335 98.4125) (width 0.6) (layer "F.Cu") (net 6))
 (segment (start 146.0675 98.2) (end 147.1225 98.2) (width 0.6) (layer "F.Cu") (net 6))
 (segment (start 145.53 97.6625) (end 146.0675 98.2) (width 0.6) (layer "F.Cu") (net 6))
 (segment (start 143.5 94.1875) (end 145.53 94.1875) (width 0.6) (layer "F.Cu") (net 8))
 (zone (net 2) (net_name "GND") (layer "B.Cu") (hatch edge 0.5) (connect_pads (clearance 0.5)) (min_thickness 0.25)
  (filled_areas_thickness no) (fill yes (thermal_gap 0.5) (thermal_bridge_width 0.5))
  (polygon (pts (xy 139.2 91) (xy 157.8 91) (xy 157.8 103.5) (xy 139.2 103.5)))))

